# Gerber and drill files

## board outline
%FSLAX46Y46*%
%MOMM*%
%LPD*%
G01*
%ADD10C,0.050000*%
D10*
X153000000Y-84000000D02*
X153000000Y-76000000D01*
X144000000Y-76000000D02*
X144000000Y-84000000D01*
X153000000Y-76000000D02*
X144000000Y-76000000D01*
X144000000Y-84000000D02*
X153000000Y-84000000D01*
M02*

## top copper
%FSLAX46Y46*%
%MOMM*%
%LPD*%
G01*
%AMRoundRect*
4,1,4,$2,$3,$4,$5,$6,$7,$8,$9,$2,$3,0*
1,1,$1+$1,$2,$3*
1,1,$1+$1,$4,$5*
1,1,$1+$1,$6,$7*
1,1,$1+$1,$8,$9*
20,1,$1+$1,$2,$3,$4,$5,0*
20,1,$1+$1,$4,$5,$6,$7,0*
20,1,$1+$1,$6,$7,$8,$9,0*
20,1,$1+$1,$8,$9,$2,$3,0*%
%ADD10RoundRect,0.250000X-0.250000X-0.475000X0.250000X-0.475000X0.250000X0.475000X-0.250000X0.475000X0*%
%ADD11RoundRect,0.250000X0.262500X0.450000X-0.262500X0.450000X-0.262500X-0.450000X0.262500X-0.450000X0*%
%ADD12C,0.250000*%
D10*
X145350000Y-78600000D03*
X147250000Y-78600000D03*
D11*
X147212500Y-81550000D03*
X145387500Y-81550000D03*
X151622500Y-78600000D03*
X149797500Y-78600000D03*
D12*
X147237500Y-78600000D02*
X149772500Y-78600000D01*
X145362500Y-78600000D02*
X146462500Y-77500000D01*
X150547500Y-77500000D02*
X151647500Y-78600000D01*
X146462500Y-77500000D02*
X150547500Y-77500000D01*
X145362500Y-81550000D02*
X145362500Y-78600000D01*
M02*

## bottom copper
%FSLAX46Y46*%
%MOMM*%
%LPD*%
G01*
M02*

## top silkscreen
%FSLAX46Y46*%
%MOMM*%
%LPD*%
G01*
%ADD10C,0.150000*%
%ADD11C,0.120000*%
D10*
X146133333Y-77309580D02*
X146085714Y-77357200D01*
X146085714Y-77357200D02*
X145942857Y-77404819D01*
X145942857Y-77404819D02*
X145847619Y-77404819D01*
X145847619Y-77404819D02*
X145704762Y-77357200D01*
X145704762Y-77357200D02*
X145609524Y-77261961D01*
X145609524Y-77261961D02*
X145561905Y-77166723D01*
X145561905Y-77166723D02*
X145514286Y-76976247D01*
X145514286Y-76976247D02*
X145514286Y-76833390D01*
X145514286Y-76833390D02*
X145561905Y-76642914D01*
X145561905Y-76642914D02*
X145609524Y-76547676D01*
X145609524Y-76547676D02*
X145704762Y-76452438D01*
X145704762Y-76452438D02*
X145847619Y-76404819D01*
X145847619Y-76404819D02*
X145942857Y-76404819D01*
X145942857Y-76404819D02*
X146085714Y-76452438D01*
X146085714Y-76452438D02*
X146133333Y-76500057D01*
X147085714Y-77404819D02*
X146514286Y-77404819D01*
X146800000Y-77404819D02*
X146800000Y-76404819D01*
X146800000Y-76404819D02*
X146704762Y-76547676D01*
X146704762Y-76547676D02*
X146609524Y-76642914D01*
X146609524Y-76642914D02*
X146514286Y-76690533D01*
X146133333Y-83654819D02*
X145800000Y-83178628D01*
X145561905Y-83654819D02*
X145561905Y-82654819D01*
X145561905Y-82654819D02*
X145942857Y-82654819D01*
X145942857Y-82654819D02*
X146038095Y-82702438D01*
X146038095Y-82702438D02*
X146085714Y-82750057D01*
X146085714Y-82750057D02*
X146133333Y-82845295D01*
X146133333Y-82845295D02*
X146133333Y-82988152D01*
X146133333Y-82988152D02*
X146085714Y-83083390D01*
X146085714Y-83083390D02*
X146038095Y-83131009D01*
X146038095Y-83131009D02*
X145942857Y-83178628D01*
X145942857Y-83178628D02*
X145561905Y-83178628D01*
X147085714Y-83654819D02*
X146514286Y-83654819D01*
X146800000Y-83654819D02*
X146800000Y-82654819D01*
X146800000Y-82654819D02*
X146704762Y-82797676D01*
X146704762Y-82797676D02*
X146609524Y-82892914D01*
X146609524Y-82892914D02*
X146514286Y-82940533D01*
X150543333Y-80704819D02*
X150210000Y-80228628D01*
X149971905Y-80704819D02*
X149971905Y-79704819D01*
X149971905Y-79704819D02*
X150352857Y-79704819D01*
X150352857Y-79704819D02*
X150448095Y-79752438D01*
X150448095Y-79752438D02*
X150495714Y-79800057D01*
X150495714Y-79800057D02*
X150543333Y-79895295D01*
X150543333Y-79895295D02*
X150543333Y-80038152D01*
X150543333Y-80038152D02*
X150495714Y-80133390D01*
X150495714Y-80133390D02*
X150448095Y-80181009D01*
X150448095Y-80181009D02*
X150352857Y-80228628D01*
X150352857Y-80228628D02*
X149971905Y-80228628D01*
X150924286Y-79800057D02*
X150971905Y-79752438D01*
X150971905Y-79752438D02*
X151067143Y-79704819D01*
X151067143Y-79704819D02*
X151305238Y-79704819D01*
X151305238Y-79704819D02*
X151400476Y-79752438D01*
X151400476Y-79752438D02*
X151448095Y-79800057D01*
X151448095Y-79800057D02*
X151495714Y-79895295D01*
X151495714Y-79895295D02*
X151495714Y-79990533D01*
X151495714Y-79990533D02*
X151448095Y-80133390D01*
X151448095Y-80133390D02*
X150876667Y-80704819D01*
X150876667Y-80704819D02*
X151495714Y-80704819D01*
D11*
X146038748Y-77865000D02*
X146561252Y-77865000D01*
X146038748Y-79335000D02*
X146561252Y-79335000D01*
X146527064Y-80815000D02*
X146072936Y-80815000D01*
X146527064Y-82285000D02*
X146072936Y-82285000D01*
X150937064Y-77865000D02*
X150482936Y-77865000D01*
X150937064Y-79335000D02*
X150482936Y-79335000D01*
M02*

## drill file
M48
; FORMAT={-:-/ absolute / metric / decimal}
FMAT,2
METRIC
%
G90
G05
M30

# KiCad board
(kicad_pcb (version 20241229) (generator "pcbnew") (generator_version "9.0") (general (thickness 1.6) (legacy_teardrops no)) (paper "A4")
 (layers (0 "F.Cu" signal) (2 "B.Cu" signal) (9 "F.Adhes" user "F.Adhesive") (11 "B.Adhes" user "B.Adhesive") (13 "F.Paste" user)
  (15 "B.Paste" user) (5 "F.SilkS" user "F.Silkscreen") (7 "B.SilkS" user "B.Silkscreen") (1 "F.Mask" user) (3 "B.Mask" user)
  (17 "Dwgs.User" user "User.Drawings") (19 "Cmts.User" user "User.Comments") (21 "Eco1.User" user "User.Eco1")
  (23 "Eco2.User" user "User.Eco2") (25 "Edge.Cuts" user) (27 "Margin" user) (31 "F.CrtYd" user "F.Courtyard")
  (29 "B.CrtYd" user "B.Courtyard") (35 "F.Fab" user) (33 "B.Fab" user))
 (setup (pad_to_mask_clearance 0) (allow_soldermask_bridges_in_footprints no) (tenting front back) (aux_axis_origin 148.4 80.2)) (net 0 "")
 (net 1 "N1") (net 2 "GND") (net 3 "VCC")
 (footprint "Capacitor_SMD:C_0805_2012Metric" (layer "F.Cu") (at 146.3 78.6)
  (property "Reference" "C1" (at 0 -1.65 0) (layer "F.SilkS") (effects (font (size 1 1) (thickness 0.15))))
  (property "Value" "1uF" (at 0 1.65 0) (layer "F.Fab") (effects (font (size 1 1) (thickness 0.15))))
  (fp_line (start -0.261252 -0.735) (end 0.261252 -0.735) (stroke (width 0.12) (type solid)) (layer "F.SilkS"))
  (fp_line (start -0.261252 0.735) (end 0.261252 0.735) (stroke (width 0.12) (type solid)) (layer "F.SilkS"))
  (pad "1" smd roundrect (at -0.95 0) (size 1 1.45) (layers "F.Cu" "F.Mask" "F.Paste") (roundrect_rratio 0.25) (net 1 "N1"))
  (pad "2" smd roundrect (at 0.95 0) (size 1 1.45) (layers "F.Cu" "F.Mask" "F.Paste") (roundrect_rratio 0.25) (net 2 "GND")))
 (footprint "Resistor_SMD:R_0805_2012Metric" (layer "F.Cu") (at 146.3 81.55 180)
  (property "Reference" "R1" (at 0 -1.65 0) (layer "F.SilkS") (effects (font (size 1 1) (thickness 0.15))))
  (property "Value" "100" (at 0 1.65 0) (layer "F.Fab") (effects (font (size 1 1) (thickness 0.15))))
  (fp_line (start -0.227064 0.735) (end 0.227064 0.735) (stroke (width 0.12) (type solid)) (layer "F.SilkS"))
  (fp_line (start -0.227064 -0.735) (end 0.227064 -0.735) (stroke (width 0.12) (type solid)) (layer "F.SilkS"))
  (pad "1" smd roundrect (at -0.9125 0 180) (size 1.025 1.4) (layers "F.Cu" "F.Mask" "F.Paste") (roundrect_rratio 0.243902) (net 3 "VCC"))
  (pad "2" smd roundrect (at 0.9125 0 180) (size 1.025 1.4) (layers "F.Cu" "F.Mask" "F.Paste") (roundrect_rratio 0.243902) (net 1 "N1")))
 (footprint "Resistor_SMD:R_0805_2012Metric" (layer "F.Cu") (at 150.71 78.6 180)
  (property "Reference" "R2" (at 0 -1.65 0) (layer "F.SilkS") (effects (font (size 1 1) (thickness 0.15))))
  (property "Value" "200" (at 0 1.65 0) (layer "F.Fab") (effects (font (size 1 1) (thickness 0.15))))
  (fp_line (start -0.227064 0.735) (end 0.227064 0.735) (stroke (width 0.12) (type solid)) (layer "F.SilkS"))
  (fp_line (start -0.227064 -0.735) (end 0.227064 -0.735) (stroke (width 0.12) (type solid)) (layer "F.SilkS"))
  (pad "1" smd roundrect (at -0.9125 0 180) (size 1.025 1.4) (layers "F.Cu" "F.Mask" "F.Paste") (roundrect_rratio 0.243902) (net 1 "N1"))
  (pad "2" smd roundrect (at 0.9125 0 180) (size 1.025 1.4) (layers "F.Cu" "F.Mask" "F.Paste") (roundrect_rratio 0.243902) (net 2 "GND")))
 (gr_line (start 153 84) (end 153 76) (stroke (width 0.05) (type solid)) (layer "Edge.Cuts"))
 (gr_line (start 144 76) (end 144 84) (stroke (width 0.05) (type solid)) (layer "Edge.Cuts"))
 (gr_line (start 153 76) (end 144 76) (stroke (width 0.05) (type solid)) (layer "Edge.Cuts"))
 (gr_line (start 144 84) (end 153 84) (stroke (width 0.05) (type solid)) (layer "Edge.Cuts"))
 (segment (start 147.2375 78.6) (end 149.7725 78.6) (width 0.25) (layer "F.Cu") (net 2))
 (segment (start 145.3625 78.6) (end 146.4625 77.5) (width 0.25) (layer "F.Cu") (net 1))
 (segment (start 150.5475 77.5) (end 151.6475 78.6) (width 0.25) (layer "F.Cu") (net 1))
 (segment (start 146.4625 77.5) (end 150.5475 77.5) (width 0.25) (layer "F.Cu") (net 1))
 (segment (start 145.3625 81.55) (end 145.3625 78.6) (width 0.25) (layer "F.Cu") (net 1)))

